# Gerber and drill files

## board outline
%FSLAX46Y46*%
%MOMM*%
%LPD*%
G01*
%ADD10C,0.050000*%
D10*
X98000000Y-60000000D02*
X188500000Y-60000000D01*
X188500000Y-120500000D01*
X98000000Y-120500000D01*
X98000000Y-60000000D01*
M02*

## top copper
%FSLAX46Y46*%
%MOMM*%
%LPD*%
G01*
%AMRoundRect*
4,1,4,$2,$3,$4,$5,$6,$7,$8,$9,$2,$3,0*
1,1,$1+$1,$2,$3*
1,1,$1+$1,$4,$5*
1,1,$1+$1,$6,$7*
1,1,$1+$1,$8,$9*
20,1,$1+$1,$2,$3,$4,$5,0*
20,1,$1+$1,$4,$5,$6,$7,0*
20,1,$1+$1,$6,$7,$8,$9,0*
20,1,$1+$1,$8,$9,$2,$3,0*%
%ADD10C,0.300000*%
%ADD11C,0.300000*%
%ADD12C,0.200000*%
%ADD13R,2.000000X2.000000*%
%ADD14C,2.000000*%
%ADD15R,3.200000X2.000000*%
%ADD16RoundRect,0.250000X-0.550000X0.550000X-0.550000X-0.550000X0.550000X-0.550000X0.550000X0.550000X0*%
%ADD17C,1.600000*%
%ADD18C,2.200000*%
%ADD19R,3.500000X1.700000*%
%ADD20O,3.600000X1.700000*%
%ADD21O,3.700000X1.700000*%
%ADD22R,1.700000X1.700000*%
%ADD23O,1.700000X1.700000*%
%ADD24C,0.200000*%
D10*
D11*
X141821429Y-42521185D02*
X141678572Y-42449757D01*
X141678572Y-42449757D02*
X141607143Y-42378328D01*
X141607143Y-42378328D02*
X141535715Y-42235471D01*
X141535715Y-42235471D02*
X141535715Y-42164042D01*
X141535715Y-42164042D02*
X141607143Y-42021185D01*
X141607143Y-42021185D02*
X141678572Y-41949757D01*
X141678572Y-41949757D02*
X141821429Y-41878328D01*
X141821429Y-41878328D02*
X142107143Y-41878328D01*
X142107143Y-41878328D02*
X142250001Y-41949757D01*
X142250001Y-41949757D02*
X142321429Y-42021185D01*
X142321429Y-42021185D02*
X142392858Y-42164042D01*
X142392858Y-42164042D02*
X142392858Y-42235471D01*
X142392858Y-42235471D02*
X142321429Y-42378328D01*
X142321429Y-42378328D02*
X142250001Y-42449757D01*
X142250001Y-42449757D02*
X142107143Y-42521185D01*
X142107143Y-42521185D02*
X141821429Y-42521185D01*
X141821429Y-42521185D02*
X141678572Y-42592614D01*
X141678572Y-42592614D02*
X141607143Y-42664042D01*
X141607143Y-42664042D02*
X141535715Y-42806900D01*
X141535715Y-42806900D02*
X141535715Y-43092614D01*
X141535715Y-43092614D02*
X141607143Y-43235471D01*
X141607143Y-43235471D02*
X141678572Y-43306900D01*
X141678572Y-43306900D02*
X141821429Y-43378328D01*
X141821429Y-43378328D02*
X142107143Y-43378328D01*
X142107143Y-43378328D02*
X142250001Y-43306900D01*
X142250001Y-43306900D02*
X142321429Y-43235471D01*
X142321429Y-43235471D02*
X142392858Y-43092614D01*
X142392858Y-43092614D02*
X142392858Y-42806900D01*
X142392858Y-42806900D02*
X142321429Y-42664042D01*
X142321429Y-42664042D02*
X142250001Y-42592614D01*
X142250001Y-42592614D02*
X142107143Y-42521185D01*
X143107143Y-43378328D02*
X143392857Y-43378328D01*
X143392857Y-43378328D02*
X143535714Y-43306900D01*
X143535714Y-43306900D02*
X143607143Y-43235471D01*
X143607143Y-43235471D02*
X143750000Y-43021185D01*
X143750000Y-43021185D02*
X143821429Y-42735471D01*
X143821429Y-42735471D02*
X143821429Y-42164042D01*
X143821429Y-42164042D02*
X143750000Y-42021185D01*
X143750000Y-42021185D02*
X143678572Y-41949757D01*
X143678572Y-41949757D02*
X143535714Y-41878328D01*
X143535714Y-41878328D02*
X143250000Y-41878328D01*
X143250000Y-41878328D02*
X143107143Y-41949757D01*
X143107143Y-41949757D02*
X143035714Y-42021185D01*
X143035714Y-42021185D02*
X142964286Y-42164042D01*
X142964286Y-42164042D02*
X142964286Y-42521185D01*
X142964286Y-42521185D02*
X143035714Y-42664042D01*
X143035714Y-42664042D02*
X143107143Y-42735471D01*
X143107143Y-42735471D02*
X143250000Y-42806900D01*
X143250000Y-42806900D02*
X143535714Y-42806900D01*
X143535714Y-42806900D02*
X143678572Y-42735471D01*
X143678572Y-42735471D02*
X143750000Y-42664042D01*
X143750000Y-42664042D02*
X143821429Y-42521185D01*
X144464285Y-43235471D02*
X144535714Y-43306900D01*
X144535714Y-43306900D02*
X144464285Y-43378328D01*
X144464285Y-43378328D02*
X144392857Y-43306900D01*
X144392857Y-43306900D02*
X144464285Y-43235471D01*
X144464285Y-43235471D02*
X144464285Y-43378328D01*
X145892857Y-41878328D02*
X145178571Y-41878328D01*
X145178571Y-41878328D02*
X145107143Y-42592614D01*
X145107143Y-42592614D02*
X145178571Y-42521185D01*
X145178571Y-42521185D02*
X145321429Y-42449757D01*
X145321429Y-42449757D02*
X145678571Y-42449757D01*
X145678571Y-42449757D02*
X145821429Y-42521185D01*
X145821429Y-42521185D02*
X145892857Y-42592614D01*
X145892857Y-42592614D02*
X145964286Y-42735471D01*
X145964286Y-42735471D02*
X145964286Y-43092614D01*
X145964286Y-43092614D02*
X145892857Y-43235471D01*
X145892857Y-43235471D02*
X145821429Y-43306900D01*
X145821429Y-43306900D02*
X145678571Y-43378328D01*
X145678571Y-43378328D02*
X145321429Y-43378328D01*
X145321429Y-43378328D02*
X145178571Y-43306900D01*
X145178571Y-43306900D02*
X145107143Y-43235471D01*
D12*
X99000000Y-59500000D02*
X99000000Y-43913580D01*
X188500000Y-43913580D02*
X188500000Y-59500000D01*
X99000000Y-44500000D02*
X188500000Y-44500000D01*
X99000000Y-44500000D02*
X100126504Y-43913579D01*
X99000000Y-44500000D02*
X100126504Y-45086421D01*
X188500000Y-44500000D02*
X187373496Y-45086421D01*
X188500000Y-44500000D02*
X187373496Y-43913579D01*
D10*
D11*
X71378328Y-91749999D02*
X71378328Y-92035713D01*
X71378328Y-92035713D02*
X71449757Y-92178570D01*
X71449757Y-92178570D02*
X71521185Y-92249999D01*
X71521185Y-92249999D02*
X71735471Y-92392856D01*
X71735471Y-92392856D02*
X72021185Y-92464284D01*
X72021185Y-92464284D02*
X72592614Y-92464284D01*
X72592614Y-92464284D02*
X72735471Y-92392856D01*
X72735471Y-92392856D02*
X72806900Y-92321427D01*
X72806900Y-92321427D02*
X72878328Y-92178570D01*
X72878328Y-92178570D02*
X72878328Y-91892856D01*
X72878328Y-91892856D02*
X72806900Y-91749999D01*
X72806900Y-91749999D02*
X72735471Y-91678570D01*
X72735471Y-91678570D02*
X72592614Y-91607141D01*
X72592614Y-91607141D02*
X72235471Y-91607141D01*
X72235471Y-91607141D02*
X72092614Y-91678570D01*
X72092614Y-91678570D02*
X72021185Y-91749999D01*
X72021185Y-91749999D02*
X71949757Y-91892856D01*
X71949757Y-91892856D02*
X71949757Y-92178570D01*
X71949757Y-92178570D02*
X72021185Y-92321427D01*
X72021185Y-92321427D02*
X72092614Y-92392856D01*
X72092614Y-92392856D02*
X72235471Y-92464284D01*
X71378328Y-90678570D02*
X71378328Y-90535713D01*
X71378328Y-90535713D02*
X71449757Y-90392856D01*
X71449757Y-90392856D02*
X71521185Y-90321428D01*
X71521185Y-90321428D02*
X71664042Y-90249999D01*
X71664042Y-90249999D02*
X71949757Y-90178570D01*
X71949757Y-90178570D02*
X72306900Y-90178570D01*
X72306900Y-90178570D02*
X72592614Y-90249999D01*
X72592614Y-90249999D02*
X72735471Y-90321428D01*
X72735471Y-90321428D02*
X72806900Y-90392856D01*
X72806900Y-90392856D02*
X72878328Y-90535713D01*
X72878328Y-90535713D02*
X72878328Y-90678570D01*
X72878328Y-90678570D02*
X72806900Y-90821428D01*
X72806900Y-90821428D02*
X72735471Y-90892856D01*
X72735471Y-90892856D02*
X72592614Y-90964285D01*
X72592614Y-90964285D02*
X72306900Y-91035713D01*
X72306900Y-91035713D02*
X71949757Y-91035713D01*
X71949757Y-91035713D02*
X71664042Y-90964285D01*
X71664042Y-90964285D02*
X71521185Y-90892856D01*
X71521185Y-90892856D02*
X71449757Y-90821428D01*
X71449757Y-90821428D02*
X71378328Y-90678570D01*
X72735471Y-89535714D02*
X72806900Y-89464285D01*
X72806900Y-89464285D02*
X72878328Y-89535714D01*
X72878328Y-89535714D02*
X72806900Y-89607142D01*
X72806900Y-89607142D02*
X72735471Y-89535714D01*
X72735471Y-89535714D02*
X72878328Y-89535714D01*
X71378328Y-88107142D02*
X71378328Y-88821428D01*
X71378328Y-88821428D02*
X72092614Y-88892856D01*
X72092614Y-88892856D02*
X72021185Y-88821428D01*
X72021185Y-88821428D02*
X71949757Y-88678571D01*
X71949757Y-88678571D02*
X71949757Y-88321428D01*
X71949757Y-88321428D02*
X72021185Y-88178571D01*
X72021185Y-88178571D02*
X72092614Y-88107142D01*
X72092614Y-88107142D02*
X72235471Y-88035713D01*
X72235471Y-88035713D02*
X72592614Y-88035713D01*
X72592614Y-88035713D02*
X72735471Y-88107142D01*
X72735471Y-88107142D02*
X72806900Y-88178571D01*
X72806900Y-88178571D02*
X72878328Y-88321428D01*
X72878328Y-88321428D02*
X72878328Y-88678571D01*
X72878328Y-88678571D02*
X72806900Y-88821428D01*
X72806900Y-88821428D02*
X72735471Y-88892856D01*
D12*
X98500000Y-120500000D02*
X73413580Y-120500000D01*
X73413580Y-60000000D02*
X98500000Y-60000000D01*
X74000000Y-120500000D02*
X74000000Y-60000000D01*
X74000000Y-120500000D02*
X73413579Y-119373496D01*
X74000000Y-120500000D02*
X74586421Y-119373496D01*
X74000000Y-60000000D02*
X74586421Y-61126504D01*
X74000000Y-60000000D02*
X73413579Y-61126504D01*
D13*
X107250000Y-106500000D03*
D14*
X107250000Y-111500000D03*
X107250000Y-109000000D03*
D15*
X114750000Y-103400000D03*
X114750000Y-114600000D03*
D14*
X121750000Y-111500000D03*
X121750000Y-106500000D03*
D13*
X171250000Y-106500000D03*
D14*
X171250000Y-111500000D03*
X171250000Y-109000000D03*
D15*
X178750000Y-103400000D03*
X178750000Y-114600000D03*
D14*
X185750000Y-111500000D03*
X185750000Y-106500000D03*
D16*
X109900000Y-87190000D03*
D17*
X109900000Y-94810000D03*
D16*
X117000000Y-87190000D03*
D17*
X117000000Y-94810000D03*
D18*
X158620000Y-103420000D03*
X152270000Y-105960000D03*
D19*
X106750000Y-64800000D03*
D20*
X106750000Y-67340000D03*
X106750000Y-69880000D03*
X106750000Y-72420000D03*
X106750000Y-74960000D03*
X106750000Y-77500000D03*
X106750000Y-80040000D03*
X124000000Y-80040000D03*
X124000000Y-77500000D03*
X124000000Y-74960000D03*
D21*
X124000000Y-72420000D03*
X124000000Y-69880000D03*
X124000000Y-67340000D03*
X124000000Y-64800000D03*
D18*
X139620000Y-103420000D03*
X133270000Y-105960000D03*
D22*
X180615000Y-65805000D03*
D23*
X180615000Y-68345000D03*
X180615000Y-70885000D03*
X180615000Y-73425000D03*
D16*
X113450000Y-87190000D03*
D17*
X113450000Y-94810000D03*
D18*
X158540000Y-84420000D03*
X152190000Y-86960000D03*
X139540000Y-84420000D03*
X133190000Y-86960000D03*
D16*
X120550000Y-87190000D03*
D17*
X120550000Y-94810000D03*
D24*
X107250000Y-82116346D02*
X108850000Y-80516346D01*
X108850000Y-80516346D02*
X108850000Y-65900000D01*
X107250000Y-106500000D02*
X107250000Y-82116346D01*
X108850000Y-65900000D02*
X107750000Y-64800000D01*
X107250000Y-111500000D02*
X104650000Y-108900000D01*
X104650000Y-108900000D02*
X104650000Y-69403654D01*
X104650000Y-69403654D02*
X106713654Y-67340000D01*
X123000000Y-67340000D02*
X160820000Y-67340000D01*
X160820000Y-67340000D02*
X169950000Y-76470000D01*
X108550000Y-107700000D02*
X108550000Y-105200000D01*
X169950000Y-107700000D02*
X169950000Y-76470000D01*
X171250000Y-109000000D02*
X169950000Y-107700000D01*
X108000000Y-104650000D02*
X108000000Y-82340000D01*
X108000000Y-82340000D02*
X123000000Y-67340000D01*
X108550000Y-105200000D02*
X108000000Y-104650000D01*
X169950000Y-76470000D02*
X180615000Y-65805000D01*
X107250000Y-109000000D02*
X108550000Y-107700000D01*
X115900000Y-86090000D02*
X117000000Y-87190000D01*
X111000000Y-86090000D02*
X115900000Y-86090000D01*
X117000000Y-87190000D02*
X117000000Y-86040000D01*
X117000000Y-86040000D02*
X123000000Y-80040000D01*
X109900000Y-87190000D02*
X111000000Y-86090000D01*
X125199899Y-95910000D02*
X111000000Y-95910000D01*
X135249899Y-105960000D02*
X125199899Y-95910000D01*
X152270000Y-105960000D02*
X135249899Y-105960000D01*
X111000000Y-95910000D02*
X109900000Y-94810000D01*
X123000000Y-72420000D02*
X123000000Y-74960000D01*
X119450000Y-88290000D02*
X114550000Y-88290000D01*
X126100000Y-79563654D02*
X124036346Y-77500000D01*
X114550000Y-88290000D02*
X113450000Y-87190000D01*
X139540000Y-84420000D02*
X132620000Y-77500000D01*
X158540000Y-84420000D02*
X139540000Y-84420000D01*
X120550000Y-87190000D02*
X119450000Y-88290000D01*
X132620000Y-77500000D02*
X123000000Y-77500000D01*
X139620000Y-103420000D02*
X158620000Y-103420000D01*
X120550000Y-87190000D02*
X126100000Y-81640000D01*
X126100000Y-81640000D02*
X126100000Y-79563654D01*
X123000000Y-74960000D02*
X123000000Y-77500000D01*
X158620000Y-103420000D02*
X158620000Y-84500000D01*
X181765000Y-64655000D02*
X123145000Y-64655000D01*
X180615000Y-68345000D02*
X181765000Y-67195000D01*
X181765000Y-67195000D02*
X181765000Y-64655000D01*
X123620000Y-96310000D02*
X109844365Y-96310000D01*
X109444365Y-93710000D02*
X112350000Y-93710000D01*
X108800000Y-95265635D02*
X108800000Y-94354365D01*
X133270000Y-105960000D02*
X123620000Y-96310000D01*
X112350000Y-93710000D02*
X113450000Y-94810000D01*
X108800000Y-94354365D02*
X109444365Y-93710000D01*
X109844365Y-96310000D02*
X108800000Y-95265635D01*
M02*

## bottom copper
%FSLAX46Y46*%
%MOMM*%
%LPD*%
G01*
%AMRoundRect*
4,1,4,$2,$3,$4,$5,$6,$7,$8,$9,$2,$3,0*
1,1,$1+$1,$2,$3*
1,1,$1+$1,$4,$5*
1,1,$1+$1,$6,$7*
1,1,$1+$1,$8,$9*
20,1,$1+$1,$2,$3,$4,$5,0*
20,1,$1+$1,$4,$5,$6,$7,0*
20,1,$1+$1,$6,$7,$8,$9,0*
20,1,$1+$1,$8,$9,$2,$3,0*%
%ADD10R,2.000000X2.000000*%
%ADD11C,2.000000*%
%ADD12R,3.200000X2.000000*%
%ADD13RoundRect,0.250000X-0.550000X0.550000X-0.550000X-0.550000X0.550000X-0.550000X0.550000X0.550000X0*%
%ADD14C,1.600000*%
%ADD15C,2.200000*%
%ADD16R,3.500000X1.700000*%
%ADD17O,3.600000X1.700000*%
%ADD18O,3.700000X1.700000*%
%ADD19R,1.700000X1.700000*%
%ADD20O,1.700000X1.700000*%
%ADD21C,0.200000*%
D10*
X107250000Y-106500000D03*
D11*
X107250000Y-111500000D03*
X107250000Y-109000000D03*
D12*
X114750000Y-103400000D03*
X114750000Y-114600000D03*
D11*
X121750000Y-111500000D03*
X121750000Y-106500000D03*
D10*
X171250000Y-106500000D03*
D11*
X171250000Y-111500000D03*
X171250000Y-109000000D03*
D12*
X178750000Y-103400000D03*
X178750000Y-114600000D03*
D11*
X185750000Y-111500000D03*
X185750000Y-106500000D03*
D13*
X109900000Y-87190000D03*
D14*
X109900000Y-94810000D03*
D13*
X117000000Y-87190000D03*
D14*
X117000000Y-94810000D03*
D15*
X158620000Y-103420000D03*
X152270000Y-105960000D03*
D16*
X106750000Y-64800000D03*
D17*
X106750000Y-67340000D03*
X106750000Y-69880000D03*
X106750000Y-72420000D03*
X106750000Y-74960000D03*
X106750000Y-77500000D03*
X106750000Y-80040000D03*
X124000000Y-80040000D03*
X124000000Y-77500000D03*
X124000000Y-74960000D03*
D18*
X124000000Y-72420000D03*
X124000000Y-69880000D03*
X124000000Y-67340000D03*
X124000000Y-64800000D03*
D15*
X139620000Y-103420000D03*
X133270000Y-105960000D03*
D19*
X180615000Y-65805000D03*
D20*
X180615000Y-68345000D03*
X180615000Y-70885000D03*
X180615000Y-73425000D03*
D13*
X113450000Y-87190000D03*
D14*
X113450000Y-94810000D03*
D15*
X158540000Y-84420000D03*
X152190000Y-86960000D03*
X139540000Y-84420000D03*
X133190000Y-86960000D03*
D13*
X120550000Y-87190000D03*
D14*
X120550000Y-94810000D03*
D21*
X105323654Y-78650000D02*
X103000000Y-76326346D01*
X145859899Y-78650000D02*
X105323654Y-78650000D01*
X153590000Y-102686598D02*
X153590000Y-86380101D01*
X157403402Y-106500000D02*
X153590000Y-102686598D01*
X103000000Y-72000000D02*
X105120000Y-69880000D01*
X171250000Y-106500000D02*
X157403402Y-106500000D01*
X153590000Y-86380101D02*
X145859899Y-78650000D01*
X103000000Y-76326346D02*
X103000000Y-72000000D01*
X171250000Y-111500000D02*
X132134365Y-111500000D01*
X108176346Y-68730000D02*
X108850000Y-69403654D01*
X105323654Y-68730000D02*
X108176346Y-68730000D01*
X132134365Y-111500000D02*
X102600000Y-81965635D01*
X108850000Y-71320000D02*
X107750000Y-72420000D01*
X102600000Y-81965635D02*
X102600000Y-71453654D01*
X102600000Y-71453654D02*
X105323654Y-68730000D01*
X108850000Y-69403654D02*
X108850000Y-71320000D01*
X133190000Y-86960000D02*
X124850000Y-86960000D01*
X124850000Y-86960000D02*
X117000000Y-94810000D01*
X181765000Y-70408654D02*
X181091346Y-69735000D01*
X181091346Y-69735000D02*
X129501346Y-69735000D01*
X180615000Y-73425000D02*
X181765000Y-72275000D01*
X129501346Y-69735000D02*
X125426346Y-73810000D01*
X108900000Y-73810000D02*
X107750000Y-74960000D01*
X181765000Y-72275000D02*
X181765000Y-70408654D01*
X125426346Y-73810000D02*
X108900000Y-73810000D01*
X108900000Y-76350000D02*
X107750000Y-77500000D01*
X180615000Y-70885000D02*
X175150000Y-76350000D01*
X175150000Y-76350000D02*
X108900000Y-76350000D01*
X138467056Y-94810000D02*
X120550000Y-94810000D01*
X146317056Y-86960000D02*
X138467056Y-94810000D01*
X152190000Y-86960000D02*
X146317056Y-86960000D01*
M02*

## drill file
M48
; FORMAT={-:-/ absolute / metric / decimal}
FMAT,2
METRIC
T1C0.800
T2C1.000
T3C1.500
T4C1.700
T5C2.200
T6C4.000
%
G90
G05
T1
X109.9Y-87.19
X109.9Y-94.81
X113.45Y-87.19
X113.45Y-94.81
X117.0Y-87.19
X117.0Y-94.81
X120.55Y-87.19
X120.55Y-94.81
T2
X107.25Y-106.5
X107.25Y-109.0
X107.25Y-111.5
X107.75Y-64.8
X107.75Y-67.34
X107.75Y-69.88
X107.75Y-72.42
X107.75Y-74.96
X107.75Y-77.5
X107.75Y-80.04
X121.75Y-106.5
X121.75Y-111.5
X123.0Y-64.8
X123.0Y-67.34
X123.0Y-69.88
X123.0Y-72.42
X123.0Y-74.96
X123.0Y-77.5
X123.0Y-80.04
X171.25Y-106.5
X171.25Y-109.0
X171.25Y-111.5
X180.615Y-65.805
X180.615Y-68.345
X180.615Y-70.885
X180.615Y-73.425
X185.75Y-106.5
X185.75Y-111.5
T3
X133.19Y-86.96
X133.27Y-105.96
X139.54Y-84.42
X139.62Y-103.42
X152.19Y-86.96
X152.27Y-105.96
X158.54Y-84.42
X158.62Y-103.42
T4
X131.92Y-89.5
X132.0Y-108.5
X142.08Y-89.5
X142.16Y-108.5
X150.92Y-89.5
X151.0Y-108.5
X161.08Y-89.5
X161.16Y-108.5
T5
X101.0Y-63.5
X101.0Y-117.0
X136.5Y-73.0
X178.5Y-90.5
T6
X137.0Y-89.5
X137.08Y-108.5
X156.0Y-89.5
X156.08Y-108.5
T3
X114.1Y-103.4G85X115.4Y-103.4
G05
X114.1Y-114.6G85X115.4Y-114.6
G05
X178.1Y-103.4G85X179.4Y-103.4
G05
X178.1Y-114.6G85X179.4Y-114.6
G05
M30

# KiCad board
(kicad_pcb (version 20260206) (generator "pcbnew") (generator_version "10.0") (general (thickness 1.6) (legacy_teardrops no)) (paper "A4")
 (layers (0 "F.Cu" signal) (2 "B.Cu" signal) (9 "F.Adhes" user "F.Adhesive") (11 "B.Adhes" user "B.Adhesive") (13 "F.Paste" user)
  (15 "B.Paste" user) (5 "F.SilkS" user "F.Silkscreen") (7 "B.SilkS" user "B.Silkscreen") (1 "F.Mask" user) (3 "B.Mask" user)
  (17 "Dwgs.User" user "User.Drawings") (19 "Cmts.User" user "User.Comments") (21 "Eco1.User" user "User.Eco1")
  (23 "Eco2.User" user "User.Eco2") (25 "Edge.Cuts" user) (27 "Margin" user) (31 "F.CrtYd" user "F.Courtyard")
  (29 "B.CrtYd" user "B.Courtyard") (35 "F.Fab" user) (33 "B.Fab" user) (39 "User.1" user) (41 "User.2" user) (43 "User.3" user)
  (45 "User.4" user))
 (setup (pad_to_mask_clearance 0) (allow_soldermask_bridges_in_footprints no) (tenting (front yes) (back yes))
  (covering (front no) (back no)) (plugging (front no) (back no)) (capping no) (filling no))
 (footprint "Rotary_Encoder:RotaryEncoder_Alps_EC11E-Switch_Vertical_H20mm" (layer "F.Cu") (at 107.25 106.5)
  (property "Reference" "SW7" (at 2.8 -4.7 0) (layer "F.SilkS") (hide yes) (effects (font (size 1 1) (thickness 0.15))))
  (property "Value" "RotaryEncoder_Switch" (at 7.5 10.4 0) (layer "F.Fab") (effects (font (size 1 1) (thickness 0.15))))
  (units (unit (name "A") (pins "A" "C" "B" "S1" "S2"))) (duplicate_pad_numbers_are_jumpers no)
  (pad "A" thru_hole rect (at 0 0) (size 2 2) (drill 1) (layers "*.Cu" "*.Mask") (remove_unused_layers no) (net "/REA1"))
  (pad "B" thru_hole circle (at 0 5) (size 2 2) (drill 1) (layers "*.Cu" "*.Mask") (remove_unused_layers no) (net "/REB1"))
  (pad "C" thru_hole circle (at 0 2.5) (size 2 2) (drill 1) (layers "*.Cu" "*.Mask") (remove_unused_layers no) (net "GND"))
  (pad "MP" thru_hole rect (at 7.5 -3.1) (size 3.2 2) (drill oval 2.8 1.5) (layers "*.Cu" "*.Mask") (remove_unused_layers no))
  (pad "MP" thru_hole rect (at 7.5 8.1) (size 3.2 2) (drill oval 2.8 1.5) (layers "*.Cu" "*.Mask") (remove_unused_layers no))
  (pad "S1" thru_hole circle (at 14.5 5) (size 2 2) (drill 1) (layers "*.Cu" "*.Mask") (remove_unused_layers no)
   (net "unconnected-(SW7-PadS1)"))
  (pad "S2" thru_hole circle (at 14.5 0) (size 2 2) (drill 1) (layers "*.Cu" "*.Mask") (remove_unused_layers no)
   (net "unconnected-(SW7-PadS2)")))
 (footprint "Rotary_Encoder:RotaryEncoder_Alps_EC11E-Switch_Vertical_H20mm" (layer "F.Cu") (at 171.25 106.5)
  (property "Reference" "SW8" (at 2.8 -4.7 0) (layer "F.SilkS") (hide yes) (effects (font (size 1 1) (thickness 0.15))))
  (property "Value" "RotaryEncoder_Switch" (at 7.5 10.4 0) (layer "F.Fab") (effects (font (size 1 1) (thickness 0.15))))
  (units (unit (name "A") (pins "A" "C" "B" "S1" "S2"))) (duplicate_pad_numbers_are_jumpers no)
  (pad "A" thru_hole rect (at 0 0) (size 2 2) (drill 1) (layers "*.Cu" "*.Mask") (remove_unused_layers no) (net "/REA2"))
  (pad "B" thru_hole circle (at 0 5) (size 2 2) (drill 1) (layers "*.Cu" "*.Mask") (remove_unused_layers no) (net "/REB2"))
  (pad "C" thru_hole circle (at 0 2.5) (size 2 2) (drill 1) (layers "*.Cu" "*.Mask") (remove_unused_layers no) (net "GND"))
  (pad "MP" thru_hole rect (at 7.5 -3.1) (size 3.2 2) (drill oval 2.8 1.5) (layers "*.Cu" "*.Mask") (remove_unused_layers no))
  (pad "MP" thru_hole rect (at 7.5 8.1) (size 3.2 2) (drill oval 2.8 1.5) (layers "*.Cu" "*.Mask") (remove_unused_layers no))
  (pad "S1" thru_hole circle (at 14.5 5) (size 2 2) (drill 1) (layers "*.Cu" "*.Mask") (remove_unused_layers no)
   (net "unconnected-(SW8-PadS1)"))
  (pad "S2" thru_hole circle (at 14.5 0) (size 2 2) (drill 1) (layers "*.Cu" "*.Mask") (remove_unused_layers no)
   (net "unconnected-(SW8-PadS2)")))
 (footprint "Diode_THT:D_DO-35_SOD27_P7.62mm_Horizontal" (layer "F.Cu") (at 109.9 87.19 -90)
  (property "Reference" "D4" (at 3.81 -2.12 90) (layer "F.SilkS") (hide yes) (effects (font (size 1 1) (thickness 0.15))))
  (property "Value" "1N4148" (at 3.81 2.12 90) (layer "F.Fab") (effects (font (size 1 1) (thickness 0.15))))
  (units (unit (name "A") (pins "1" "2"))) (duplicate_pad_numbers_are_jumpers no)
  (pad "1" thru_hole roundrect (at 0 0 270) (size 1.6 1.6) (drill 0.8) (layers "*.Cu" "*.Mask") (remove_unused_layers no)
   (roundrect_rratio 0.15625) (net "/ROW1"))
  (pad "2" thru_hole circle (at 7.62 0 270) (size 1.6 1.6) (drill 0.8) (layers "*.Cu" "*.Mask") (remove_unused_layers no) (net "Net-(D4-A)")))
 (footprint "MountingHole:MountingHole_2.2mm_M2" (layer "F.Cu") (at 136.5 73)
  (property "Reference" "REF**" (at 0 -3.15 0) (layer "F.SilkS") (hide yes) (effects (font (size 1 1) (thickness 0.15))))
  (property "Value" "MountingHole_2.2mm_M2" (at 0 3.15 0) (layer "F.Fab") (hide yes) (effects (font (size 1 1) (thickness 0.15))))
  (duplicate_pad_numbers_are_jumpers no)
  (pad "" np_thru_hole circle (at 0 0) (size 2.2 2.2) (drill 2.2) (layers "*.Cu" "*.Mask")))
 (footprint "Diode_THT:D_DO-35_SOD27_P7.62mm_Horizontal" (layer "F.Cu") (at 117 87.19 -90)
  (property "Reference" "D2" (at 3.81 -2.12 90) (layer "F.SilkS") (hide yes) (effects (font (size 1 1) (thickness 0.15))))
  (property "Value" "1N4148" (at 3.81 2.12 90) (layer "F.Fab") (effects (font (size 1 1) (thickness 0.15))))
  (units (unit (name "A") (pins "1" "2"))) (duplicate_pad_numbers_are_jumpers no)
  (pad "1" thru_hole roundrect (at 0 0 270) (size 1.6 1.6) (drill 0.8) (layers "*.Cu" "*.Mask") (remove_unused_layers no)
   (roundrect_rratio 0.15625) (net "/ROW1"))
  (pad "2" thru_hole circle (at 7.62 0 270) (size 1.6 1.6) (drill 0.8) (layers "*.Cu" "*.Mask") (remove_unused_layers no) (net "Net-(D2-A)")))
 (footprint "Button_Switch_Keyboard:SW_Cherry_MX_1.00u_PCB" (layer "F.Cu") (at 158.62 103.42)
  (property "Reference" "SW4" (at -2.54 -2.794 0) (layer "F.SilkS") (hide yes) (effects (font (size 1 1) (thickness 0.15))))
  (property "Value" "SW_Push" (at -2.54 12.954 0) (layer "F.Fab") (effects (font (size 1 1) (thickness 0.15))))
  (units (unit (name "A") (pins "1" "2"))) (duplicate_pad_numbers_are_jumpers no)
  (pad "" np_thru_hole circle (at -7.62 5.08) (size 1.7 1.7) (drill 1.7) (layers "*.Cu" "*.Mask"))
  (pad "" np_thru_hole circle (at -2.54 5.08) (size 4 4) (drill 4) (layers "*.Cu" "*.Mask"))
  (pad "" np_thru_hole circle (at 2.54 5.08) (size 1.7 1.7) (drill 1.7) (layers "*.Cu" "*.Mask"))
  (pad "1" thru_hole circle (at 0 0) (size 2.2 2.2) (drill 1.5) (layers "*.Cu" "*.Mask") (remove_unused_layers no) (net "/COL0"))
  (pad "2" thru_hole circle (at -6.35 2.54) (size 2.2 2.2) (drill 1.5) (layers "*.Cu" "*.Mask") (remove_unused_layers no) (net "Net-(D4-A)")))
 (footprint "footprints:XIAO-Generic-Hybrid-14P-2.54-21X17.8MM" (layer "F.Cu") (at 115.375 72.42)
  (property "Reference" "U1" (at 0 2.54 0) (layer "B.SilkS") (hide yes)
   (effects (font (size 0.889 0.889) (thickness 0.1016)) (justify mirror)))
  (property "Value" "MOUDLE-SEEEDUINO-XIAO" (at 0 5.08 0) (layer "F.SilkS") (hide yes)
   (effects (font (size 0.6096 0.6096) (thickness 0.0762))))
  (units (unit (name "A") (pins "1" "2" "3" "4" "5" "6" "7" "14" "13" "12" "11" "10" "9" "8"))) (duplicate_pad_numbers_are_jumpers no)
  (pad "1" thru_hole rect (at -7.625 -7.62) (size 3.5 1.7) (drill 1 (offset -1 0)) (layers "*.Cu" "*.Mask") (remove_unused_layers no)
   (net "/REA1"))
  (pad "2" thru_hole oval (at -7.625 -5.08) (size 3.6 1.7) (drill 1 (offset -1 0)) (layers "*.Cu" "*.Mask") (remove_unused_layers no)
   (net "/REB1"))
  (pad "3" thru_hole oval (at -7.625 -2.54) (size 3.6 1.7) (drill 1 (offset -1 0)) (layers "*.Cu" "*.Mask") (remove_unused_layers no)
   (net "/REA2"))
  (pad "4" thru_hole oval (at -7.625 0) (size 3.6 1.7) (drill 1 (offset -1 0)) (layers "*.Cu" "*.Mask") (remove_unused_layers no)
   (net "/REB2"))
  (pad "5" thru_hole oval (at -7.625 2.54) (size 3.6 1.7) (drill 1 (offset -1 0)) (layers "*.Cu" "*.Mask") (remove_unused_layers no)
   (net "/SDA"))
  (pad "6" thru_hole oval (at -7.625 5.08 180) (size 3.6 1.7) (drill 1 (offset 1 0)) (layers "*.Cu" "*.Mask") (remove_unused_layers no)
   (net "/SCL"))
  (pad "7" thru_hole oval (at -7.625 7.62) (size 3.6 1.7) (drill 1 (offset -1 0)) (layers "*.Cu" "*.Mask") (remove_unused_layers no)
   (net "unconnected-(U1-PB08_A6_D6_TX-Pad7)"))
  (pad "8" thru_hole oval (at 7.625 7.62) (size 3.6 1.7) (drill 1 (offset 1 0)) (layers "*.Cu" "*.Mask") (remove_unused_layers no)
   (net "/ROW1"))
  (pad "9" thru_hole oval (at 7.625 5.08) (size 3.6 1.7) (drill 1 (offset 1 0)) (layers "*.Cu" "*.Mask") (remove_unused_layers no)
   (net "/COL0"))
  (pad "10" thru_hole oval (at 7.625 2.54) (size 3.6 1.7) (drill 1 (offset 1 0)) (layers "*.Cu" "*.Mask") (remove_unused_layers no)
   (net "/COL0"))
  (pad "11" thru_hole oval (at 7.625 0) (size 3.7 1.7) (drill 1 (offset 1 0)) (layers "*.Cu" "*.Mask") (remove_unused_layers no)
   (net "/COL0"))
  (pad "12" thru_hole oval (at 7.625 -2.54) (size 3.7 1.7) (drill 1 (offset 1 0)) (layers "*.Cu" "*.Mask") (remove_unused_layers no)
   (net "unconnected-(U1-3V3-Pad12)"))
  (pad "13" thru_hole oval (at 7.625 -5.08) (size 3.7 1.7) (drill 1 (offset 1 0)) (layers "*.Cu" "*.Mask") (remove_unused_layers no)
   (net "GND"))
  (pad "14" thru_hole oval (at 7.625 -7.62) (size 3.7 1.7) (drill 1 (offset 1 0)) (layers "*.Cu" "*.Mask") (remove_unused_layers no)
   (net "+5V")))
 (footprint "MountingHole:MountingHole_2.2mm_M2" (layer "F.Cu") (at 101 117)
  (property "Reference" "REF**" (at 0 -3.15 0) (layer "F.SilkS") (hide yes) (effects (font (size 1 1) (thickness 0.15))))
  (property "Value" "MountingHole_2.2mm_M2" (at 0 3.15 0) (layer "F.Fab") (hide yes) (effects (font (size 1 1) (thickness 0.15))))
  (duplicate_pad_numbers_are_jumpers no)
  (pad "" np_thru_hole circle (at 0 0) (size 2.2 2.2) (drill 2.2) (layers "*.Cu" "*.Mask")))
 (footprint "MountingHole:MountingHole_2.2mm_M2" (layer "F.Cu") (at 178.5 90.5)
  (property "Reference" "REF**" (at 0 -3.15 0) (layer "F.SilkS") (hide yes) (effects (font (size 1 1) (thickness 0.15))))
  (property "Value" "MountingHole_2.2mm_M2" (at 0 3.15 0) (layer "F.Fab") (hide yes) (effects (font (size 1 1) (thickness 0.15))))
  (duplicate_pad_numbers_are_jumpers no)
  (pad "" np_thru_hole circle (at 0 0) (size 2.2 2.2) (drill 2.2) (layers "*.Cu" "*.Mask")))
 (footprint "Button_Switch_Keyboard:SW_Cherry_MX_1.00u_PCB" (layer "F.Cu") (at 139.62 103.42)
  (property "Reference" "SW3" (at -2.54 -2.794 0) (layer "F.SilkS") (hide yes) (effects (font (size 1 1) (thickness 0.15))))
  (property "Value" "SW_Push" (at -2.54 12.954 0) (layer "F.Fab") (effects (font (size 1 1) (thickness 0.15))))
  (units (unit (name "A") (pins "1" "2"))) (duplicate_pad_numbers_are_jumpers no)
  (pad "" np_thru_hole circle (at -7.62 5.08) (size 1.7 1.7) (drill 1.7) (layers "*.Cu" "*.Mask"))
  (pad "" np_thru_hole circle (at -2.54 5.08) (size 4 4) (drill 4) (layers "*.Cu" "*.Mask"))
  (pad "" np_thru_hole circle (at 2.54 5.08) (size 1.7 1.7) (drill 1.7) (layers "*.Cu" "*.Mask"))
  (pad "1" thru_hole circle (at 0 0) (size 2.2 2.2) (drill 1.5) (layers "*.Cu" "*.Mask") (remove_unused_layers no) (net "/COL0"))
  (pad "2" thru_hole circle (at -6.35 2.54) (size 2.2 2.2) (drill 1.5) (layers "*.Cu" "*.Mask") (remove_unused_layers no) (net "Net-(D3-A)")))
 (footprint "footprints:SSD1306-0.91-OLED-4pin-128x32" (layer "F.Cu") (at 144.115 63.615)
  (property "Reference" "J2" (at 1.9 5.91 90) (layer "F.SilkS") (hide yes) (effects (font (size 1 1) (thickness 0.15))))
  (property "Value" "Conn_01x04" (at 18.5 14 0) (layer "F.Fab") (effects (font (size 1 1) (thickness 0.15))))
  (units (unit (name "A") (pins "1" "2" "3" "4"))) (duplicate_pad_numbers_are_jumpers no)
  (pad "1" thru_hole rect (at 36.5 2.19) (size 1.7 1.7) (drill 1) (layers "*.Cu" "*.Mask") (remove_unused_layers no) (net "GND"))
  (pad "2" thru_hole oval (at 36.5 4.73) (size 1.7 1.7) (drill 1) (layers "*.Cu" "*.Mask") (remove_unused_layers no) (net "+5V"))
  (pad "3" thru_hole oval (at 36.5 7.27) (size 1.7 1.7) (drill 1) (layers "*.Cu" "*.Mask") (remove_unused_layers no) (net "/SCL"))
  (pad "4" thru_hole oval (at 36.5 9.81) (size 1.7 1.7) (drill 1) (layers "*.Cu" "*.Mask") (remove_unused_layers no) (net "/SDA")))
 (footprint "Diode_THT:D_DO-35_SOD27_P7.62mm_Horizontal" (layer "F.Cu") (at 113.45 87.19 -90)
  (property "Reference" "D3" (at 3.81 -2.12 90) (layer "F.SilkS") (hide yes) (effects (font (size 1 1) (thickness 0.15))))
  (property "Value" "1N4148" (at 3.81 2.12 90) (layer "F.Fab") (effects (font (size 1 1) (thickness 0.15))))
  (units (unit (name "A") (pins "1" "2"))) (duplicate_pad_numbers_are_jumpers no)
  (pad "1" thru_hole roundrect (at 0 0 270) (size 1.6 1.6) (drill 0.8) (layers "*.Cu" "*.Mask") (remove_unused_layers no)
   (roundrect_rratio 0.15625) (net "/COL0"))
  (pad "2" thru_hole circle (at 7.62 0 270) (size 1.6 1.6) (drill 0.8) (layers "*.Cu" "*.Mask") (remove_unused_layers no) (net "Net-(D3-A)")))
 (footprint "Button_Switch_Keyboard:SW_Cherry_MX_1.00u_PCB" (layer "F.Cu") (at 158.54 84.42)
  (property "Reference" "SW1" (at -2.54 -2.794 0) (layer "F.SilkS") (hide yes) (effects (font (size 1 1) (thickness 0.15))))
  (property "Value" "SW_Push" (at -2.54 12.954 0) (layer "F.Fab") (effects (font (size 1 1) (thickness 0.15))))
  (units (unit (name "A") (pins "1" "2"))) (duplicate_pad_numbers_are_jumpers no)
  (pad "" np_thru_hole circle (at -7.62 5.08) (size 1.7 1.7) (drill 1.7) (layers "*.Cu" "*.Mask"))
  (pad "" np_thru_hole circle (at -2.54 5.08) (size 4 4) (drill 4) (layers "*.Cu" "*.Mask"))
  (pad "" np_thru_hole circle (at 2.54 5.08) (size 1.7 1.7) (drill 1.7) (layers "*.Cu" "*.Mask"))
  (pad "1" thru_hole circle (at 0 0) (size 2.2 2.2) (drill 1.5) (layers "*.Cu" "*.Mask") (remove_unused_layers no) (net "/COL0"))
  (pad "2" thru_hole circle (at -6.35 2.54) (size 2.2 2.2) (drill 1.5) (layers "*.Cu" "*.Mask") (remove_unused_layers no) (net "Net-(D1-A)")))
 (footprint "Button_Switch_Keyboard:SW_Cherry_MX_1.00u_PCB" (layer "F.Cu") (at 139.54 84.42)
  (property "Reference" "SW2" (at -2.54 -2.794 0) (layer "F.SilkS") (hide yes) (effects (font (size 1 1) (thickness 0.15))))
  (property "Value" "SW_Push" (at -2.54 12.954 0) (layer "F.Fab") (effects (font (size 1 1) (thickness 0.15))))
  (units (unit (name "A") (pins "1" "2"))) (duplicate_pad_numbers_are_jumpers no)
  (pad "" np_thru_hole circle (at -7.62 5.08) (size 1.7 1.7) (drill 1.7) (layers "*.Cu" "*.Mask"))
  (pad "" np_thru_hole circle (at -2.54 5.08) (size 4 4) (drill 4) (layers "*.Cu" "*.Mask"))
  (pad "" np_thru_hole circle (at 2.54 5.08) (size 1.7 1.7) (drill 1.7) (layers "*.Cu" "*.Mask"))
  (pad "1" thru_hole circle (at 0 0) (size 2.2 2.2) (drill 1.5) (layers "*.Cu" "*.Mask") (remove_unused_layers no) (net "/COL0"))
  (pad "2" thru_hole circle (at -6.35 2.54) (size 2.2 2.2) (drill 1.5) (layers "*.Cu" "*.Mask") (remove_unused_layers no) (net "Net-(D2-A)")))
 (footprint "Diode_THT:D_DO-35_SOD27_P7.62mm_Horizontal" (layer "F.Cu") (at 120.55 87.19 -90)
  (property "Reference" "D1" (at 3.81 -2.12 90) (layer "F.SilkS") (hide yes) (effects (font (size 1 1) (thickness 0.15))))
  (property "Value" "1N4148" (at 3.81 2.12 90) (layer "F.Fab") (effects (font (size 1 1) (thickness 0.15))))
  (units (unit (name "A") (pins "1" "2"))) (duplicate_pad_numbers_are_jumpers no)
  (pad "1" thru_hole roundrect (at 0 0 270) (size 1.6 1.6) (drill 0.8) (layers "*.Cu" "*.Mask") (remove_unused_layers no)
   (roundrect_rratio 0.15625) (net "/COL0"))
  (pad "2" thru_hole circle (at 7.62 0 270) (size 1.6 1.6) (drill 0.8) (layers "*.Cu" "*.Mask") (remove_unused_layers no) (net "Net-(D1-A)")))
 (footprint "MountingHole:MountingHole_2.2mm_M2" (layer "F.Cu") (at 101 63.5)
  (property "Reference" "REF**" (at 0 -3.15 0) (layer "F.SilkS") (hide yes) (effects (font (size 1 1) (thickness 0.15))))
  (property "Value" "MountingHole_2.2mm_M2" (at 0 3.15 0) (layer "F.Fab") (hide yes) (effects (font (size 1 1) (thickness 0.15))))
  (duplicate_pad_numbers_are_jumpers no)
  (pad "" np_thru_hole circle (at 0 0) (size 2.2 2.2) (drill 2.2) (layers "*.Cu" "*.Mask")))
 (gr_rect (start 98 60) (end 188.5 120.5) (stroke (width 0.05) (type default)) (fill no) (layer "Edge.Cuts"))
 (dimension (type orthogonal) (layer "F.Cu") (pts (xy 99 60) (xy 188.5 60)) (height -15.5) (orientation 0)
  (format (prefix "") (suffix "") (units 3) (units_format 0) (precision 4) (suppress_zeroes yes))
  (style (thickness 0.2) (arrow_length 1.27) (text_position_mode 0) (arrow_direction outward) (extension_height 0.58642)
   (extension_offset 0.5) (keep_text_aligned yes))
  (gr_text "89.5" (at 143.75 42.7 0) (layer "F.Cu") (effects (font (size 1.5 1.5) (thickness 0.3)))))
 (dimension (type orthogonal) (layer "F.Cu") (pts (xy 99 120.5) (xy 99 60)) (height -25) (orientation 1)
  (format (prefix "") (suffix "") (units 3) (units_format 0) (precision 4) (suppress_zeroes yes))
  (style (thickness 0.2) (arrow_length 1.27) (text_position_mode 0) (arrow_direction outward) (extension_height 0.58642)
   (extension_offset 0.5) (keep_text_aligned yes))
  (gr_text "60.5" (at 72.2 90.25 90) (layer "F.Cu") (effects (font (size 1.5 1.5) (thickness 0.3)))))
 (segment (start 107.25 82.116346) (end 108.85 80.516346) (width 0.2) (layer "F.Cu") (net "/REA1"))
 (segment (start 108.85 80.516346) (end 108.85 65.9) (width 0.2) (layer "F.Cu") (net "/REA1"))
 (segment (start 107.25 106.5) (end 107.25 82.116346) (width 0.2) (layer "F.Cu") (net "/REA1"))
 (segment (start 108.85 65.9) (end 107.75 64.8) (width 0.2) (layer "F.Cu") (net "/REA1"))
 (segment (start 107.25 111.5) (end 104.65 108.9) (width 0.2) (layer "F.Cu") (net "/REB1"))
 (segment (start 104.65 108.9) (end 104.65 69.403654) (width 0.2) (layer "F.Cu") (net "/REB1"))
 (segment (start 104.65 69.403654) (end 106.713654 67.34) (width 0.2) (layer "F.Cu") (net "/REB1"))
 (segment (start 123 67.34) (end 160.82 67.34) (width 0.2) (layer "F.Cu") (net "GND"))
 (segment (start 160.82 67.34) (end 169.95 76.47) (width 0.2) (layer "F.Cu") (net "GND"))
 (segment (start 108.55 107.7) (end 108.55 105.2) (width 0.2) (layer "F.Cu") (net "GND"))
 (segment (start 169.95 107.7) (end 169.95 76.47) (width 0.2) (layer "F.Cu") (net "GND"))
 (segment (start 171.25 109) (end 169.95 107.7) (width 0.2) (layer "F.Cu") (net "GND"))
 (segment (start 108 104.65) (end 108 82.34) (width 0.2) (layer "F.Cu") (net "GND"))
 (segment (start 108 82.34) (end 123 67.34) (width 0.2) (layer "F.Cu") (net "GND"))
 (segment (start 108.55 105.2) (end 108 104.65) (width 0.2) (layer "F.Cu") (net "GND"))
 (segment (start 169.95 76.47) (end 180.615 65.805) (width 0.2) (layer "F.Cu") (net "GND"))
 (segment (start 107.25 109) (end 108.55 107.7) (width 0.2) (layer "F.Cu") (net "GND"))
 (segment (start 105.323654 78.65) (end 103 76.326346) (width 0.2) (layer "B.Cu") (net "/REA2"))
 (segment (start 145.859899 78.65) (end 105.323654 78.65) (width 0.2) (layer "B.Cu") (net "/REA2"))
 (segment (start 153.59 102.686598) (end 153.59 86.380101) (width 0.2) (layer "B.Cu") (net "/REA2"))
 (segment (start 157.403402 106.5) (end 153.59 102.686598) (width 0.2) (layer "B.Cu") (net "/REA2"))
 (segment (start 103 72) (end 105.12 69.88) (width 0.2) (layer "B.Cu") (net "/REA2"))
 (segment (start 171.25 106.5) (end 157.403402 106.5) (width 0.2) (layer "B.Cu") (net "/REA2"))
 (segment (start 153.59 86.380101) (end 145.859899 78.65) (width 0.2) (layer "B.Cu") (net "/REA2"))
 (segment (start 103 76.326346) (end 103 72) (width 0.2) (layer "B.Cu") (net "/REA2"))
 (segment (start 171.25 111.5) (end 132.134365 111.5) (width 0.2) (layer "B.Cu") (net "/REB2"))
 (segment (start 108.176346 68.73) (end 108.85 69.403654) (width 0.2) (layer "B.Cu") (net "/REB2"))
 (segment (start 105.323654 68.73) (end 108.176346 68.73) (width 0.2) (layer "B.Cu") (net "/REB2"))
 (segment (start 132.134365 111.5) (end 102.6 81.965635) (width 0.2) (layer "B.Cu") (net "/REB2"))
 (segment (start 108.85 71.32) (end 107.75 72.42) (width 0.2) (layer "B.Cu") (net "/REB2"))
 (segment (start 102.6 81.965635) (end 102.6 71.453654) (width 0.2) (layer "B.Cu") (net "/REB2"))
 (segment (start 102.6 71.453654) (end 105.323654 68.73) (width 0.2) (layer "B.Cu") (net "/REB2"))
 (segment (start 108.85 69.403654) (end 108.85 71.32) (width 0.2) (layer "B.Cu") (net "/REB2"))
 (segment (start 115.9 86.09) (end 117 87.19) (width 0.2) (layer "F.Cu") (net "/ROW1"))
 (segment (start 111 86.09) (end 115.9 86.09) (width 0.2) (layer "F.Cu") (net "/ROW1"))
 (segment (start 117 87.19) (end 117 86.04) (width 0.2) (layer "F.Cu") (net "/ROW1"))
 (segment (start 117 86.04) (end 123 80.04) (width 0.2) (layer "F.Cu") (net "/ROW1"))
 (segment (start 109.9 87.19) (end 111 86.09) (width 0.2) (layer "F.Cu") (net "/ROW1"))
 (segment (start 125.199899 95.91) (end 111 95.91) (width 0.2) (layer "F.Cu") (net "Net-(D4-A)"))
 (segment (start 135.249899 105.96) (end 125.199899 95.91) (width 0.2) (layer "F.Cu") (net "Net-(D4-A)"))
 (segment (start 152.27 105.96) (end 135.249899 105.96) (width 0.2) (layer "F.Cu") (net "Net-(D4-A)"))
 (segment (start 111 95.91) (end 109.9 94.81) (width 0.2) (layer "F.Cu") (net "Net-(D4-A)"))
 (segment (start 133.19 86.96) (end 124.85 86.96) (width 0.2) (layer "B.Cu") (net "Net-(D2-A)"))
 (segment (start 124.85 86.96) (end 117 94.81) (width 0.2) (layer "B.Cu") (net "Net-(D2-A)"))
 (segment (start 123 72.42) (end 123 74.96) (width 0.2) (layer "F.Cu") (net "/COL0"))
 (segment (start 119.45 88.29) (end 114.55 88.29) (width 0.2) (layer "F.Cu") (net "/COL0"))
 (segment (start 126.1 79.563654) (end 124.036346 77.5) (width 0.2) (layer "F.Cu") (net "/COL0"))
 (segment (start 114.55 88.29) (end 113.45 87.19) (width 0.2) (layer "F.Cu") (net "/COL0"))
 (segment (start 139.54 84.42) (end 132.62 77.5) (width 0.2) (layer "F.Cu") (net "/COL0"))
 (segment (start 158.54 84.42) (end 139.54 84.42) (width 0.2) (layer "F.Cu") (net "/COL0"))
 (segment (start 120.55 87.19) (end 119.45 88.29) (width 0.2) (layer "F.Cu") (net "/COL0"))
 (segment (start 132.62 77.5) (end 123 77.5) (width 0.2) (layer "F.Cu") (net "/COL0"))
 (segment (start 139.62 103.42) (end 158.62 103.42) (width 0.2) (layer "F.Cu") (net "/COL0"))
 (segment (start 120.55 87.19) (end 126.1 81.64) (width 0.2) (layer "F.Cu") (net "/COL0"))
 (segment (start 126.1 81.64) (end 126.1 79.563654) (width 0.2) (layer "F.Cu") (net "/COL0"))
 (segment (start 123 74.96) (end 123 77.5) (width 0.2) (layer "F.Cu") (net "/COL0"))
 (segment (start 158.62 103.42) (end 158.62 84.5) (width 0.2) (layer "F.Cu") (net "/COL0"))
 (segment (start 181.765 70.408654) (end 181.091346 69.735) (width 0.2) (layer "B.Cu") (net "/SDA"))
 (segment (start 181.091346 69.735) (end 129.501346 69.735) (width 0.2) (layer "B.Cu") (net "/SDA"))
 (segment (start 180.615 73.425) (end 181.765 72.275) (width 0.2) (layer "B.Cu") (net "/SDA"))
 (segment (start 129.501346 69.735) (end 125.426346 73.81) (width 0.2) (layer "B.Cu") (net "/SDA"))
 (segment (start 108.9 73.81) (end 107.75 74.96) (width 0.2) (layer "B.Cu") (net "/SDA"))
 (segment (start 181.765 72.275) (end 181.765 70.408654) (width 0.2) (layer "B.Cu") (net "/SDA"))
 (segment (start 125.426346 73.81) (end 108.9 73.81) (width 0.2) (layer "B.Cu") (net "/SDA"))
 (segment (start 108.9 76.35) (end 107.75 77.5) (width 0.2) (layer "B.Cu") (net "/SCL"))
 (segment (start 180.615 70.885) (end 175.15 76.35) (width 0.2) (layer "B.Cu") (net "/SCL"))
 (segment (start 175.15 76.35) (end 108.9 76.35) (width 0.2) (layer "B.Cu") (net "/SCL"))
 (segment (start 181.765 64.655) (end 123.145 64.655) (width 0.2) (layer "F.Cu") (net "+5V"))
 (segment (start 180.615 68.345) (end 181.765 67.195) (width 0.2) (layer "F.Cu") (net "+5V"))
 (segment (start 181.765 67.195) (end 181.765 64.655) (width 0.2) (layer "F.Cu") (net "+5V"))
 (segment (start 123.62 96.31) (end 109.844365 96.31) (width 0.2) (layer "F.Cu") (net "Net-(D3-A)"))
 (segment (start 109.444365 93.71) (end 112.35 93.71) (width 0.2) (layer "F.Cu") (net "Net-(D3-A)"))
 (segment (start 108.8 95.265635) (end 108.8 94.354365) (width 0.2) (layer "F.Cu") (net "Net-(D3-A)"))
 (segment (start 133.27 105.96) (end 123.62 96.31) (width 0.2) (layer "F.Cu") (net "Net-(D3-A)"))
 (segment (start 112.35 93.71) (end 113.45 94.81) (width 0.2) (layer "F.Cu") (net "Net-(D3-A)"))
 (segment (start 108.8 94.354365) (end 109.444365 93.71) (width 0.2) (layer "F.Cu") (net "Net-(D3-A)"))
 (segment (start 109.844365 96.31) (end 108.8 95.265635) (width 0.2) (layer "F.Cu") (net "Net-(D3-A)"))
 (segment (start 138.467056 94.81) (end 120.55 94.81) (width 0.2) (layer "B.Cu") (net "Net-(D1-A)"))
 (segment (start 146.317056 86.96) (end 138.467056 94.81) (width 0.2) (layer "B.Cu") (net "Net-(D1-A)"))
 (segment (start 152.19 86.96) (end 146.317056 86.96) (width 0.2) (layer "B.Cu") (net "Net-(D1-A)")))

